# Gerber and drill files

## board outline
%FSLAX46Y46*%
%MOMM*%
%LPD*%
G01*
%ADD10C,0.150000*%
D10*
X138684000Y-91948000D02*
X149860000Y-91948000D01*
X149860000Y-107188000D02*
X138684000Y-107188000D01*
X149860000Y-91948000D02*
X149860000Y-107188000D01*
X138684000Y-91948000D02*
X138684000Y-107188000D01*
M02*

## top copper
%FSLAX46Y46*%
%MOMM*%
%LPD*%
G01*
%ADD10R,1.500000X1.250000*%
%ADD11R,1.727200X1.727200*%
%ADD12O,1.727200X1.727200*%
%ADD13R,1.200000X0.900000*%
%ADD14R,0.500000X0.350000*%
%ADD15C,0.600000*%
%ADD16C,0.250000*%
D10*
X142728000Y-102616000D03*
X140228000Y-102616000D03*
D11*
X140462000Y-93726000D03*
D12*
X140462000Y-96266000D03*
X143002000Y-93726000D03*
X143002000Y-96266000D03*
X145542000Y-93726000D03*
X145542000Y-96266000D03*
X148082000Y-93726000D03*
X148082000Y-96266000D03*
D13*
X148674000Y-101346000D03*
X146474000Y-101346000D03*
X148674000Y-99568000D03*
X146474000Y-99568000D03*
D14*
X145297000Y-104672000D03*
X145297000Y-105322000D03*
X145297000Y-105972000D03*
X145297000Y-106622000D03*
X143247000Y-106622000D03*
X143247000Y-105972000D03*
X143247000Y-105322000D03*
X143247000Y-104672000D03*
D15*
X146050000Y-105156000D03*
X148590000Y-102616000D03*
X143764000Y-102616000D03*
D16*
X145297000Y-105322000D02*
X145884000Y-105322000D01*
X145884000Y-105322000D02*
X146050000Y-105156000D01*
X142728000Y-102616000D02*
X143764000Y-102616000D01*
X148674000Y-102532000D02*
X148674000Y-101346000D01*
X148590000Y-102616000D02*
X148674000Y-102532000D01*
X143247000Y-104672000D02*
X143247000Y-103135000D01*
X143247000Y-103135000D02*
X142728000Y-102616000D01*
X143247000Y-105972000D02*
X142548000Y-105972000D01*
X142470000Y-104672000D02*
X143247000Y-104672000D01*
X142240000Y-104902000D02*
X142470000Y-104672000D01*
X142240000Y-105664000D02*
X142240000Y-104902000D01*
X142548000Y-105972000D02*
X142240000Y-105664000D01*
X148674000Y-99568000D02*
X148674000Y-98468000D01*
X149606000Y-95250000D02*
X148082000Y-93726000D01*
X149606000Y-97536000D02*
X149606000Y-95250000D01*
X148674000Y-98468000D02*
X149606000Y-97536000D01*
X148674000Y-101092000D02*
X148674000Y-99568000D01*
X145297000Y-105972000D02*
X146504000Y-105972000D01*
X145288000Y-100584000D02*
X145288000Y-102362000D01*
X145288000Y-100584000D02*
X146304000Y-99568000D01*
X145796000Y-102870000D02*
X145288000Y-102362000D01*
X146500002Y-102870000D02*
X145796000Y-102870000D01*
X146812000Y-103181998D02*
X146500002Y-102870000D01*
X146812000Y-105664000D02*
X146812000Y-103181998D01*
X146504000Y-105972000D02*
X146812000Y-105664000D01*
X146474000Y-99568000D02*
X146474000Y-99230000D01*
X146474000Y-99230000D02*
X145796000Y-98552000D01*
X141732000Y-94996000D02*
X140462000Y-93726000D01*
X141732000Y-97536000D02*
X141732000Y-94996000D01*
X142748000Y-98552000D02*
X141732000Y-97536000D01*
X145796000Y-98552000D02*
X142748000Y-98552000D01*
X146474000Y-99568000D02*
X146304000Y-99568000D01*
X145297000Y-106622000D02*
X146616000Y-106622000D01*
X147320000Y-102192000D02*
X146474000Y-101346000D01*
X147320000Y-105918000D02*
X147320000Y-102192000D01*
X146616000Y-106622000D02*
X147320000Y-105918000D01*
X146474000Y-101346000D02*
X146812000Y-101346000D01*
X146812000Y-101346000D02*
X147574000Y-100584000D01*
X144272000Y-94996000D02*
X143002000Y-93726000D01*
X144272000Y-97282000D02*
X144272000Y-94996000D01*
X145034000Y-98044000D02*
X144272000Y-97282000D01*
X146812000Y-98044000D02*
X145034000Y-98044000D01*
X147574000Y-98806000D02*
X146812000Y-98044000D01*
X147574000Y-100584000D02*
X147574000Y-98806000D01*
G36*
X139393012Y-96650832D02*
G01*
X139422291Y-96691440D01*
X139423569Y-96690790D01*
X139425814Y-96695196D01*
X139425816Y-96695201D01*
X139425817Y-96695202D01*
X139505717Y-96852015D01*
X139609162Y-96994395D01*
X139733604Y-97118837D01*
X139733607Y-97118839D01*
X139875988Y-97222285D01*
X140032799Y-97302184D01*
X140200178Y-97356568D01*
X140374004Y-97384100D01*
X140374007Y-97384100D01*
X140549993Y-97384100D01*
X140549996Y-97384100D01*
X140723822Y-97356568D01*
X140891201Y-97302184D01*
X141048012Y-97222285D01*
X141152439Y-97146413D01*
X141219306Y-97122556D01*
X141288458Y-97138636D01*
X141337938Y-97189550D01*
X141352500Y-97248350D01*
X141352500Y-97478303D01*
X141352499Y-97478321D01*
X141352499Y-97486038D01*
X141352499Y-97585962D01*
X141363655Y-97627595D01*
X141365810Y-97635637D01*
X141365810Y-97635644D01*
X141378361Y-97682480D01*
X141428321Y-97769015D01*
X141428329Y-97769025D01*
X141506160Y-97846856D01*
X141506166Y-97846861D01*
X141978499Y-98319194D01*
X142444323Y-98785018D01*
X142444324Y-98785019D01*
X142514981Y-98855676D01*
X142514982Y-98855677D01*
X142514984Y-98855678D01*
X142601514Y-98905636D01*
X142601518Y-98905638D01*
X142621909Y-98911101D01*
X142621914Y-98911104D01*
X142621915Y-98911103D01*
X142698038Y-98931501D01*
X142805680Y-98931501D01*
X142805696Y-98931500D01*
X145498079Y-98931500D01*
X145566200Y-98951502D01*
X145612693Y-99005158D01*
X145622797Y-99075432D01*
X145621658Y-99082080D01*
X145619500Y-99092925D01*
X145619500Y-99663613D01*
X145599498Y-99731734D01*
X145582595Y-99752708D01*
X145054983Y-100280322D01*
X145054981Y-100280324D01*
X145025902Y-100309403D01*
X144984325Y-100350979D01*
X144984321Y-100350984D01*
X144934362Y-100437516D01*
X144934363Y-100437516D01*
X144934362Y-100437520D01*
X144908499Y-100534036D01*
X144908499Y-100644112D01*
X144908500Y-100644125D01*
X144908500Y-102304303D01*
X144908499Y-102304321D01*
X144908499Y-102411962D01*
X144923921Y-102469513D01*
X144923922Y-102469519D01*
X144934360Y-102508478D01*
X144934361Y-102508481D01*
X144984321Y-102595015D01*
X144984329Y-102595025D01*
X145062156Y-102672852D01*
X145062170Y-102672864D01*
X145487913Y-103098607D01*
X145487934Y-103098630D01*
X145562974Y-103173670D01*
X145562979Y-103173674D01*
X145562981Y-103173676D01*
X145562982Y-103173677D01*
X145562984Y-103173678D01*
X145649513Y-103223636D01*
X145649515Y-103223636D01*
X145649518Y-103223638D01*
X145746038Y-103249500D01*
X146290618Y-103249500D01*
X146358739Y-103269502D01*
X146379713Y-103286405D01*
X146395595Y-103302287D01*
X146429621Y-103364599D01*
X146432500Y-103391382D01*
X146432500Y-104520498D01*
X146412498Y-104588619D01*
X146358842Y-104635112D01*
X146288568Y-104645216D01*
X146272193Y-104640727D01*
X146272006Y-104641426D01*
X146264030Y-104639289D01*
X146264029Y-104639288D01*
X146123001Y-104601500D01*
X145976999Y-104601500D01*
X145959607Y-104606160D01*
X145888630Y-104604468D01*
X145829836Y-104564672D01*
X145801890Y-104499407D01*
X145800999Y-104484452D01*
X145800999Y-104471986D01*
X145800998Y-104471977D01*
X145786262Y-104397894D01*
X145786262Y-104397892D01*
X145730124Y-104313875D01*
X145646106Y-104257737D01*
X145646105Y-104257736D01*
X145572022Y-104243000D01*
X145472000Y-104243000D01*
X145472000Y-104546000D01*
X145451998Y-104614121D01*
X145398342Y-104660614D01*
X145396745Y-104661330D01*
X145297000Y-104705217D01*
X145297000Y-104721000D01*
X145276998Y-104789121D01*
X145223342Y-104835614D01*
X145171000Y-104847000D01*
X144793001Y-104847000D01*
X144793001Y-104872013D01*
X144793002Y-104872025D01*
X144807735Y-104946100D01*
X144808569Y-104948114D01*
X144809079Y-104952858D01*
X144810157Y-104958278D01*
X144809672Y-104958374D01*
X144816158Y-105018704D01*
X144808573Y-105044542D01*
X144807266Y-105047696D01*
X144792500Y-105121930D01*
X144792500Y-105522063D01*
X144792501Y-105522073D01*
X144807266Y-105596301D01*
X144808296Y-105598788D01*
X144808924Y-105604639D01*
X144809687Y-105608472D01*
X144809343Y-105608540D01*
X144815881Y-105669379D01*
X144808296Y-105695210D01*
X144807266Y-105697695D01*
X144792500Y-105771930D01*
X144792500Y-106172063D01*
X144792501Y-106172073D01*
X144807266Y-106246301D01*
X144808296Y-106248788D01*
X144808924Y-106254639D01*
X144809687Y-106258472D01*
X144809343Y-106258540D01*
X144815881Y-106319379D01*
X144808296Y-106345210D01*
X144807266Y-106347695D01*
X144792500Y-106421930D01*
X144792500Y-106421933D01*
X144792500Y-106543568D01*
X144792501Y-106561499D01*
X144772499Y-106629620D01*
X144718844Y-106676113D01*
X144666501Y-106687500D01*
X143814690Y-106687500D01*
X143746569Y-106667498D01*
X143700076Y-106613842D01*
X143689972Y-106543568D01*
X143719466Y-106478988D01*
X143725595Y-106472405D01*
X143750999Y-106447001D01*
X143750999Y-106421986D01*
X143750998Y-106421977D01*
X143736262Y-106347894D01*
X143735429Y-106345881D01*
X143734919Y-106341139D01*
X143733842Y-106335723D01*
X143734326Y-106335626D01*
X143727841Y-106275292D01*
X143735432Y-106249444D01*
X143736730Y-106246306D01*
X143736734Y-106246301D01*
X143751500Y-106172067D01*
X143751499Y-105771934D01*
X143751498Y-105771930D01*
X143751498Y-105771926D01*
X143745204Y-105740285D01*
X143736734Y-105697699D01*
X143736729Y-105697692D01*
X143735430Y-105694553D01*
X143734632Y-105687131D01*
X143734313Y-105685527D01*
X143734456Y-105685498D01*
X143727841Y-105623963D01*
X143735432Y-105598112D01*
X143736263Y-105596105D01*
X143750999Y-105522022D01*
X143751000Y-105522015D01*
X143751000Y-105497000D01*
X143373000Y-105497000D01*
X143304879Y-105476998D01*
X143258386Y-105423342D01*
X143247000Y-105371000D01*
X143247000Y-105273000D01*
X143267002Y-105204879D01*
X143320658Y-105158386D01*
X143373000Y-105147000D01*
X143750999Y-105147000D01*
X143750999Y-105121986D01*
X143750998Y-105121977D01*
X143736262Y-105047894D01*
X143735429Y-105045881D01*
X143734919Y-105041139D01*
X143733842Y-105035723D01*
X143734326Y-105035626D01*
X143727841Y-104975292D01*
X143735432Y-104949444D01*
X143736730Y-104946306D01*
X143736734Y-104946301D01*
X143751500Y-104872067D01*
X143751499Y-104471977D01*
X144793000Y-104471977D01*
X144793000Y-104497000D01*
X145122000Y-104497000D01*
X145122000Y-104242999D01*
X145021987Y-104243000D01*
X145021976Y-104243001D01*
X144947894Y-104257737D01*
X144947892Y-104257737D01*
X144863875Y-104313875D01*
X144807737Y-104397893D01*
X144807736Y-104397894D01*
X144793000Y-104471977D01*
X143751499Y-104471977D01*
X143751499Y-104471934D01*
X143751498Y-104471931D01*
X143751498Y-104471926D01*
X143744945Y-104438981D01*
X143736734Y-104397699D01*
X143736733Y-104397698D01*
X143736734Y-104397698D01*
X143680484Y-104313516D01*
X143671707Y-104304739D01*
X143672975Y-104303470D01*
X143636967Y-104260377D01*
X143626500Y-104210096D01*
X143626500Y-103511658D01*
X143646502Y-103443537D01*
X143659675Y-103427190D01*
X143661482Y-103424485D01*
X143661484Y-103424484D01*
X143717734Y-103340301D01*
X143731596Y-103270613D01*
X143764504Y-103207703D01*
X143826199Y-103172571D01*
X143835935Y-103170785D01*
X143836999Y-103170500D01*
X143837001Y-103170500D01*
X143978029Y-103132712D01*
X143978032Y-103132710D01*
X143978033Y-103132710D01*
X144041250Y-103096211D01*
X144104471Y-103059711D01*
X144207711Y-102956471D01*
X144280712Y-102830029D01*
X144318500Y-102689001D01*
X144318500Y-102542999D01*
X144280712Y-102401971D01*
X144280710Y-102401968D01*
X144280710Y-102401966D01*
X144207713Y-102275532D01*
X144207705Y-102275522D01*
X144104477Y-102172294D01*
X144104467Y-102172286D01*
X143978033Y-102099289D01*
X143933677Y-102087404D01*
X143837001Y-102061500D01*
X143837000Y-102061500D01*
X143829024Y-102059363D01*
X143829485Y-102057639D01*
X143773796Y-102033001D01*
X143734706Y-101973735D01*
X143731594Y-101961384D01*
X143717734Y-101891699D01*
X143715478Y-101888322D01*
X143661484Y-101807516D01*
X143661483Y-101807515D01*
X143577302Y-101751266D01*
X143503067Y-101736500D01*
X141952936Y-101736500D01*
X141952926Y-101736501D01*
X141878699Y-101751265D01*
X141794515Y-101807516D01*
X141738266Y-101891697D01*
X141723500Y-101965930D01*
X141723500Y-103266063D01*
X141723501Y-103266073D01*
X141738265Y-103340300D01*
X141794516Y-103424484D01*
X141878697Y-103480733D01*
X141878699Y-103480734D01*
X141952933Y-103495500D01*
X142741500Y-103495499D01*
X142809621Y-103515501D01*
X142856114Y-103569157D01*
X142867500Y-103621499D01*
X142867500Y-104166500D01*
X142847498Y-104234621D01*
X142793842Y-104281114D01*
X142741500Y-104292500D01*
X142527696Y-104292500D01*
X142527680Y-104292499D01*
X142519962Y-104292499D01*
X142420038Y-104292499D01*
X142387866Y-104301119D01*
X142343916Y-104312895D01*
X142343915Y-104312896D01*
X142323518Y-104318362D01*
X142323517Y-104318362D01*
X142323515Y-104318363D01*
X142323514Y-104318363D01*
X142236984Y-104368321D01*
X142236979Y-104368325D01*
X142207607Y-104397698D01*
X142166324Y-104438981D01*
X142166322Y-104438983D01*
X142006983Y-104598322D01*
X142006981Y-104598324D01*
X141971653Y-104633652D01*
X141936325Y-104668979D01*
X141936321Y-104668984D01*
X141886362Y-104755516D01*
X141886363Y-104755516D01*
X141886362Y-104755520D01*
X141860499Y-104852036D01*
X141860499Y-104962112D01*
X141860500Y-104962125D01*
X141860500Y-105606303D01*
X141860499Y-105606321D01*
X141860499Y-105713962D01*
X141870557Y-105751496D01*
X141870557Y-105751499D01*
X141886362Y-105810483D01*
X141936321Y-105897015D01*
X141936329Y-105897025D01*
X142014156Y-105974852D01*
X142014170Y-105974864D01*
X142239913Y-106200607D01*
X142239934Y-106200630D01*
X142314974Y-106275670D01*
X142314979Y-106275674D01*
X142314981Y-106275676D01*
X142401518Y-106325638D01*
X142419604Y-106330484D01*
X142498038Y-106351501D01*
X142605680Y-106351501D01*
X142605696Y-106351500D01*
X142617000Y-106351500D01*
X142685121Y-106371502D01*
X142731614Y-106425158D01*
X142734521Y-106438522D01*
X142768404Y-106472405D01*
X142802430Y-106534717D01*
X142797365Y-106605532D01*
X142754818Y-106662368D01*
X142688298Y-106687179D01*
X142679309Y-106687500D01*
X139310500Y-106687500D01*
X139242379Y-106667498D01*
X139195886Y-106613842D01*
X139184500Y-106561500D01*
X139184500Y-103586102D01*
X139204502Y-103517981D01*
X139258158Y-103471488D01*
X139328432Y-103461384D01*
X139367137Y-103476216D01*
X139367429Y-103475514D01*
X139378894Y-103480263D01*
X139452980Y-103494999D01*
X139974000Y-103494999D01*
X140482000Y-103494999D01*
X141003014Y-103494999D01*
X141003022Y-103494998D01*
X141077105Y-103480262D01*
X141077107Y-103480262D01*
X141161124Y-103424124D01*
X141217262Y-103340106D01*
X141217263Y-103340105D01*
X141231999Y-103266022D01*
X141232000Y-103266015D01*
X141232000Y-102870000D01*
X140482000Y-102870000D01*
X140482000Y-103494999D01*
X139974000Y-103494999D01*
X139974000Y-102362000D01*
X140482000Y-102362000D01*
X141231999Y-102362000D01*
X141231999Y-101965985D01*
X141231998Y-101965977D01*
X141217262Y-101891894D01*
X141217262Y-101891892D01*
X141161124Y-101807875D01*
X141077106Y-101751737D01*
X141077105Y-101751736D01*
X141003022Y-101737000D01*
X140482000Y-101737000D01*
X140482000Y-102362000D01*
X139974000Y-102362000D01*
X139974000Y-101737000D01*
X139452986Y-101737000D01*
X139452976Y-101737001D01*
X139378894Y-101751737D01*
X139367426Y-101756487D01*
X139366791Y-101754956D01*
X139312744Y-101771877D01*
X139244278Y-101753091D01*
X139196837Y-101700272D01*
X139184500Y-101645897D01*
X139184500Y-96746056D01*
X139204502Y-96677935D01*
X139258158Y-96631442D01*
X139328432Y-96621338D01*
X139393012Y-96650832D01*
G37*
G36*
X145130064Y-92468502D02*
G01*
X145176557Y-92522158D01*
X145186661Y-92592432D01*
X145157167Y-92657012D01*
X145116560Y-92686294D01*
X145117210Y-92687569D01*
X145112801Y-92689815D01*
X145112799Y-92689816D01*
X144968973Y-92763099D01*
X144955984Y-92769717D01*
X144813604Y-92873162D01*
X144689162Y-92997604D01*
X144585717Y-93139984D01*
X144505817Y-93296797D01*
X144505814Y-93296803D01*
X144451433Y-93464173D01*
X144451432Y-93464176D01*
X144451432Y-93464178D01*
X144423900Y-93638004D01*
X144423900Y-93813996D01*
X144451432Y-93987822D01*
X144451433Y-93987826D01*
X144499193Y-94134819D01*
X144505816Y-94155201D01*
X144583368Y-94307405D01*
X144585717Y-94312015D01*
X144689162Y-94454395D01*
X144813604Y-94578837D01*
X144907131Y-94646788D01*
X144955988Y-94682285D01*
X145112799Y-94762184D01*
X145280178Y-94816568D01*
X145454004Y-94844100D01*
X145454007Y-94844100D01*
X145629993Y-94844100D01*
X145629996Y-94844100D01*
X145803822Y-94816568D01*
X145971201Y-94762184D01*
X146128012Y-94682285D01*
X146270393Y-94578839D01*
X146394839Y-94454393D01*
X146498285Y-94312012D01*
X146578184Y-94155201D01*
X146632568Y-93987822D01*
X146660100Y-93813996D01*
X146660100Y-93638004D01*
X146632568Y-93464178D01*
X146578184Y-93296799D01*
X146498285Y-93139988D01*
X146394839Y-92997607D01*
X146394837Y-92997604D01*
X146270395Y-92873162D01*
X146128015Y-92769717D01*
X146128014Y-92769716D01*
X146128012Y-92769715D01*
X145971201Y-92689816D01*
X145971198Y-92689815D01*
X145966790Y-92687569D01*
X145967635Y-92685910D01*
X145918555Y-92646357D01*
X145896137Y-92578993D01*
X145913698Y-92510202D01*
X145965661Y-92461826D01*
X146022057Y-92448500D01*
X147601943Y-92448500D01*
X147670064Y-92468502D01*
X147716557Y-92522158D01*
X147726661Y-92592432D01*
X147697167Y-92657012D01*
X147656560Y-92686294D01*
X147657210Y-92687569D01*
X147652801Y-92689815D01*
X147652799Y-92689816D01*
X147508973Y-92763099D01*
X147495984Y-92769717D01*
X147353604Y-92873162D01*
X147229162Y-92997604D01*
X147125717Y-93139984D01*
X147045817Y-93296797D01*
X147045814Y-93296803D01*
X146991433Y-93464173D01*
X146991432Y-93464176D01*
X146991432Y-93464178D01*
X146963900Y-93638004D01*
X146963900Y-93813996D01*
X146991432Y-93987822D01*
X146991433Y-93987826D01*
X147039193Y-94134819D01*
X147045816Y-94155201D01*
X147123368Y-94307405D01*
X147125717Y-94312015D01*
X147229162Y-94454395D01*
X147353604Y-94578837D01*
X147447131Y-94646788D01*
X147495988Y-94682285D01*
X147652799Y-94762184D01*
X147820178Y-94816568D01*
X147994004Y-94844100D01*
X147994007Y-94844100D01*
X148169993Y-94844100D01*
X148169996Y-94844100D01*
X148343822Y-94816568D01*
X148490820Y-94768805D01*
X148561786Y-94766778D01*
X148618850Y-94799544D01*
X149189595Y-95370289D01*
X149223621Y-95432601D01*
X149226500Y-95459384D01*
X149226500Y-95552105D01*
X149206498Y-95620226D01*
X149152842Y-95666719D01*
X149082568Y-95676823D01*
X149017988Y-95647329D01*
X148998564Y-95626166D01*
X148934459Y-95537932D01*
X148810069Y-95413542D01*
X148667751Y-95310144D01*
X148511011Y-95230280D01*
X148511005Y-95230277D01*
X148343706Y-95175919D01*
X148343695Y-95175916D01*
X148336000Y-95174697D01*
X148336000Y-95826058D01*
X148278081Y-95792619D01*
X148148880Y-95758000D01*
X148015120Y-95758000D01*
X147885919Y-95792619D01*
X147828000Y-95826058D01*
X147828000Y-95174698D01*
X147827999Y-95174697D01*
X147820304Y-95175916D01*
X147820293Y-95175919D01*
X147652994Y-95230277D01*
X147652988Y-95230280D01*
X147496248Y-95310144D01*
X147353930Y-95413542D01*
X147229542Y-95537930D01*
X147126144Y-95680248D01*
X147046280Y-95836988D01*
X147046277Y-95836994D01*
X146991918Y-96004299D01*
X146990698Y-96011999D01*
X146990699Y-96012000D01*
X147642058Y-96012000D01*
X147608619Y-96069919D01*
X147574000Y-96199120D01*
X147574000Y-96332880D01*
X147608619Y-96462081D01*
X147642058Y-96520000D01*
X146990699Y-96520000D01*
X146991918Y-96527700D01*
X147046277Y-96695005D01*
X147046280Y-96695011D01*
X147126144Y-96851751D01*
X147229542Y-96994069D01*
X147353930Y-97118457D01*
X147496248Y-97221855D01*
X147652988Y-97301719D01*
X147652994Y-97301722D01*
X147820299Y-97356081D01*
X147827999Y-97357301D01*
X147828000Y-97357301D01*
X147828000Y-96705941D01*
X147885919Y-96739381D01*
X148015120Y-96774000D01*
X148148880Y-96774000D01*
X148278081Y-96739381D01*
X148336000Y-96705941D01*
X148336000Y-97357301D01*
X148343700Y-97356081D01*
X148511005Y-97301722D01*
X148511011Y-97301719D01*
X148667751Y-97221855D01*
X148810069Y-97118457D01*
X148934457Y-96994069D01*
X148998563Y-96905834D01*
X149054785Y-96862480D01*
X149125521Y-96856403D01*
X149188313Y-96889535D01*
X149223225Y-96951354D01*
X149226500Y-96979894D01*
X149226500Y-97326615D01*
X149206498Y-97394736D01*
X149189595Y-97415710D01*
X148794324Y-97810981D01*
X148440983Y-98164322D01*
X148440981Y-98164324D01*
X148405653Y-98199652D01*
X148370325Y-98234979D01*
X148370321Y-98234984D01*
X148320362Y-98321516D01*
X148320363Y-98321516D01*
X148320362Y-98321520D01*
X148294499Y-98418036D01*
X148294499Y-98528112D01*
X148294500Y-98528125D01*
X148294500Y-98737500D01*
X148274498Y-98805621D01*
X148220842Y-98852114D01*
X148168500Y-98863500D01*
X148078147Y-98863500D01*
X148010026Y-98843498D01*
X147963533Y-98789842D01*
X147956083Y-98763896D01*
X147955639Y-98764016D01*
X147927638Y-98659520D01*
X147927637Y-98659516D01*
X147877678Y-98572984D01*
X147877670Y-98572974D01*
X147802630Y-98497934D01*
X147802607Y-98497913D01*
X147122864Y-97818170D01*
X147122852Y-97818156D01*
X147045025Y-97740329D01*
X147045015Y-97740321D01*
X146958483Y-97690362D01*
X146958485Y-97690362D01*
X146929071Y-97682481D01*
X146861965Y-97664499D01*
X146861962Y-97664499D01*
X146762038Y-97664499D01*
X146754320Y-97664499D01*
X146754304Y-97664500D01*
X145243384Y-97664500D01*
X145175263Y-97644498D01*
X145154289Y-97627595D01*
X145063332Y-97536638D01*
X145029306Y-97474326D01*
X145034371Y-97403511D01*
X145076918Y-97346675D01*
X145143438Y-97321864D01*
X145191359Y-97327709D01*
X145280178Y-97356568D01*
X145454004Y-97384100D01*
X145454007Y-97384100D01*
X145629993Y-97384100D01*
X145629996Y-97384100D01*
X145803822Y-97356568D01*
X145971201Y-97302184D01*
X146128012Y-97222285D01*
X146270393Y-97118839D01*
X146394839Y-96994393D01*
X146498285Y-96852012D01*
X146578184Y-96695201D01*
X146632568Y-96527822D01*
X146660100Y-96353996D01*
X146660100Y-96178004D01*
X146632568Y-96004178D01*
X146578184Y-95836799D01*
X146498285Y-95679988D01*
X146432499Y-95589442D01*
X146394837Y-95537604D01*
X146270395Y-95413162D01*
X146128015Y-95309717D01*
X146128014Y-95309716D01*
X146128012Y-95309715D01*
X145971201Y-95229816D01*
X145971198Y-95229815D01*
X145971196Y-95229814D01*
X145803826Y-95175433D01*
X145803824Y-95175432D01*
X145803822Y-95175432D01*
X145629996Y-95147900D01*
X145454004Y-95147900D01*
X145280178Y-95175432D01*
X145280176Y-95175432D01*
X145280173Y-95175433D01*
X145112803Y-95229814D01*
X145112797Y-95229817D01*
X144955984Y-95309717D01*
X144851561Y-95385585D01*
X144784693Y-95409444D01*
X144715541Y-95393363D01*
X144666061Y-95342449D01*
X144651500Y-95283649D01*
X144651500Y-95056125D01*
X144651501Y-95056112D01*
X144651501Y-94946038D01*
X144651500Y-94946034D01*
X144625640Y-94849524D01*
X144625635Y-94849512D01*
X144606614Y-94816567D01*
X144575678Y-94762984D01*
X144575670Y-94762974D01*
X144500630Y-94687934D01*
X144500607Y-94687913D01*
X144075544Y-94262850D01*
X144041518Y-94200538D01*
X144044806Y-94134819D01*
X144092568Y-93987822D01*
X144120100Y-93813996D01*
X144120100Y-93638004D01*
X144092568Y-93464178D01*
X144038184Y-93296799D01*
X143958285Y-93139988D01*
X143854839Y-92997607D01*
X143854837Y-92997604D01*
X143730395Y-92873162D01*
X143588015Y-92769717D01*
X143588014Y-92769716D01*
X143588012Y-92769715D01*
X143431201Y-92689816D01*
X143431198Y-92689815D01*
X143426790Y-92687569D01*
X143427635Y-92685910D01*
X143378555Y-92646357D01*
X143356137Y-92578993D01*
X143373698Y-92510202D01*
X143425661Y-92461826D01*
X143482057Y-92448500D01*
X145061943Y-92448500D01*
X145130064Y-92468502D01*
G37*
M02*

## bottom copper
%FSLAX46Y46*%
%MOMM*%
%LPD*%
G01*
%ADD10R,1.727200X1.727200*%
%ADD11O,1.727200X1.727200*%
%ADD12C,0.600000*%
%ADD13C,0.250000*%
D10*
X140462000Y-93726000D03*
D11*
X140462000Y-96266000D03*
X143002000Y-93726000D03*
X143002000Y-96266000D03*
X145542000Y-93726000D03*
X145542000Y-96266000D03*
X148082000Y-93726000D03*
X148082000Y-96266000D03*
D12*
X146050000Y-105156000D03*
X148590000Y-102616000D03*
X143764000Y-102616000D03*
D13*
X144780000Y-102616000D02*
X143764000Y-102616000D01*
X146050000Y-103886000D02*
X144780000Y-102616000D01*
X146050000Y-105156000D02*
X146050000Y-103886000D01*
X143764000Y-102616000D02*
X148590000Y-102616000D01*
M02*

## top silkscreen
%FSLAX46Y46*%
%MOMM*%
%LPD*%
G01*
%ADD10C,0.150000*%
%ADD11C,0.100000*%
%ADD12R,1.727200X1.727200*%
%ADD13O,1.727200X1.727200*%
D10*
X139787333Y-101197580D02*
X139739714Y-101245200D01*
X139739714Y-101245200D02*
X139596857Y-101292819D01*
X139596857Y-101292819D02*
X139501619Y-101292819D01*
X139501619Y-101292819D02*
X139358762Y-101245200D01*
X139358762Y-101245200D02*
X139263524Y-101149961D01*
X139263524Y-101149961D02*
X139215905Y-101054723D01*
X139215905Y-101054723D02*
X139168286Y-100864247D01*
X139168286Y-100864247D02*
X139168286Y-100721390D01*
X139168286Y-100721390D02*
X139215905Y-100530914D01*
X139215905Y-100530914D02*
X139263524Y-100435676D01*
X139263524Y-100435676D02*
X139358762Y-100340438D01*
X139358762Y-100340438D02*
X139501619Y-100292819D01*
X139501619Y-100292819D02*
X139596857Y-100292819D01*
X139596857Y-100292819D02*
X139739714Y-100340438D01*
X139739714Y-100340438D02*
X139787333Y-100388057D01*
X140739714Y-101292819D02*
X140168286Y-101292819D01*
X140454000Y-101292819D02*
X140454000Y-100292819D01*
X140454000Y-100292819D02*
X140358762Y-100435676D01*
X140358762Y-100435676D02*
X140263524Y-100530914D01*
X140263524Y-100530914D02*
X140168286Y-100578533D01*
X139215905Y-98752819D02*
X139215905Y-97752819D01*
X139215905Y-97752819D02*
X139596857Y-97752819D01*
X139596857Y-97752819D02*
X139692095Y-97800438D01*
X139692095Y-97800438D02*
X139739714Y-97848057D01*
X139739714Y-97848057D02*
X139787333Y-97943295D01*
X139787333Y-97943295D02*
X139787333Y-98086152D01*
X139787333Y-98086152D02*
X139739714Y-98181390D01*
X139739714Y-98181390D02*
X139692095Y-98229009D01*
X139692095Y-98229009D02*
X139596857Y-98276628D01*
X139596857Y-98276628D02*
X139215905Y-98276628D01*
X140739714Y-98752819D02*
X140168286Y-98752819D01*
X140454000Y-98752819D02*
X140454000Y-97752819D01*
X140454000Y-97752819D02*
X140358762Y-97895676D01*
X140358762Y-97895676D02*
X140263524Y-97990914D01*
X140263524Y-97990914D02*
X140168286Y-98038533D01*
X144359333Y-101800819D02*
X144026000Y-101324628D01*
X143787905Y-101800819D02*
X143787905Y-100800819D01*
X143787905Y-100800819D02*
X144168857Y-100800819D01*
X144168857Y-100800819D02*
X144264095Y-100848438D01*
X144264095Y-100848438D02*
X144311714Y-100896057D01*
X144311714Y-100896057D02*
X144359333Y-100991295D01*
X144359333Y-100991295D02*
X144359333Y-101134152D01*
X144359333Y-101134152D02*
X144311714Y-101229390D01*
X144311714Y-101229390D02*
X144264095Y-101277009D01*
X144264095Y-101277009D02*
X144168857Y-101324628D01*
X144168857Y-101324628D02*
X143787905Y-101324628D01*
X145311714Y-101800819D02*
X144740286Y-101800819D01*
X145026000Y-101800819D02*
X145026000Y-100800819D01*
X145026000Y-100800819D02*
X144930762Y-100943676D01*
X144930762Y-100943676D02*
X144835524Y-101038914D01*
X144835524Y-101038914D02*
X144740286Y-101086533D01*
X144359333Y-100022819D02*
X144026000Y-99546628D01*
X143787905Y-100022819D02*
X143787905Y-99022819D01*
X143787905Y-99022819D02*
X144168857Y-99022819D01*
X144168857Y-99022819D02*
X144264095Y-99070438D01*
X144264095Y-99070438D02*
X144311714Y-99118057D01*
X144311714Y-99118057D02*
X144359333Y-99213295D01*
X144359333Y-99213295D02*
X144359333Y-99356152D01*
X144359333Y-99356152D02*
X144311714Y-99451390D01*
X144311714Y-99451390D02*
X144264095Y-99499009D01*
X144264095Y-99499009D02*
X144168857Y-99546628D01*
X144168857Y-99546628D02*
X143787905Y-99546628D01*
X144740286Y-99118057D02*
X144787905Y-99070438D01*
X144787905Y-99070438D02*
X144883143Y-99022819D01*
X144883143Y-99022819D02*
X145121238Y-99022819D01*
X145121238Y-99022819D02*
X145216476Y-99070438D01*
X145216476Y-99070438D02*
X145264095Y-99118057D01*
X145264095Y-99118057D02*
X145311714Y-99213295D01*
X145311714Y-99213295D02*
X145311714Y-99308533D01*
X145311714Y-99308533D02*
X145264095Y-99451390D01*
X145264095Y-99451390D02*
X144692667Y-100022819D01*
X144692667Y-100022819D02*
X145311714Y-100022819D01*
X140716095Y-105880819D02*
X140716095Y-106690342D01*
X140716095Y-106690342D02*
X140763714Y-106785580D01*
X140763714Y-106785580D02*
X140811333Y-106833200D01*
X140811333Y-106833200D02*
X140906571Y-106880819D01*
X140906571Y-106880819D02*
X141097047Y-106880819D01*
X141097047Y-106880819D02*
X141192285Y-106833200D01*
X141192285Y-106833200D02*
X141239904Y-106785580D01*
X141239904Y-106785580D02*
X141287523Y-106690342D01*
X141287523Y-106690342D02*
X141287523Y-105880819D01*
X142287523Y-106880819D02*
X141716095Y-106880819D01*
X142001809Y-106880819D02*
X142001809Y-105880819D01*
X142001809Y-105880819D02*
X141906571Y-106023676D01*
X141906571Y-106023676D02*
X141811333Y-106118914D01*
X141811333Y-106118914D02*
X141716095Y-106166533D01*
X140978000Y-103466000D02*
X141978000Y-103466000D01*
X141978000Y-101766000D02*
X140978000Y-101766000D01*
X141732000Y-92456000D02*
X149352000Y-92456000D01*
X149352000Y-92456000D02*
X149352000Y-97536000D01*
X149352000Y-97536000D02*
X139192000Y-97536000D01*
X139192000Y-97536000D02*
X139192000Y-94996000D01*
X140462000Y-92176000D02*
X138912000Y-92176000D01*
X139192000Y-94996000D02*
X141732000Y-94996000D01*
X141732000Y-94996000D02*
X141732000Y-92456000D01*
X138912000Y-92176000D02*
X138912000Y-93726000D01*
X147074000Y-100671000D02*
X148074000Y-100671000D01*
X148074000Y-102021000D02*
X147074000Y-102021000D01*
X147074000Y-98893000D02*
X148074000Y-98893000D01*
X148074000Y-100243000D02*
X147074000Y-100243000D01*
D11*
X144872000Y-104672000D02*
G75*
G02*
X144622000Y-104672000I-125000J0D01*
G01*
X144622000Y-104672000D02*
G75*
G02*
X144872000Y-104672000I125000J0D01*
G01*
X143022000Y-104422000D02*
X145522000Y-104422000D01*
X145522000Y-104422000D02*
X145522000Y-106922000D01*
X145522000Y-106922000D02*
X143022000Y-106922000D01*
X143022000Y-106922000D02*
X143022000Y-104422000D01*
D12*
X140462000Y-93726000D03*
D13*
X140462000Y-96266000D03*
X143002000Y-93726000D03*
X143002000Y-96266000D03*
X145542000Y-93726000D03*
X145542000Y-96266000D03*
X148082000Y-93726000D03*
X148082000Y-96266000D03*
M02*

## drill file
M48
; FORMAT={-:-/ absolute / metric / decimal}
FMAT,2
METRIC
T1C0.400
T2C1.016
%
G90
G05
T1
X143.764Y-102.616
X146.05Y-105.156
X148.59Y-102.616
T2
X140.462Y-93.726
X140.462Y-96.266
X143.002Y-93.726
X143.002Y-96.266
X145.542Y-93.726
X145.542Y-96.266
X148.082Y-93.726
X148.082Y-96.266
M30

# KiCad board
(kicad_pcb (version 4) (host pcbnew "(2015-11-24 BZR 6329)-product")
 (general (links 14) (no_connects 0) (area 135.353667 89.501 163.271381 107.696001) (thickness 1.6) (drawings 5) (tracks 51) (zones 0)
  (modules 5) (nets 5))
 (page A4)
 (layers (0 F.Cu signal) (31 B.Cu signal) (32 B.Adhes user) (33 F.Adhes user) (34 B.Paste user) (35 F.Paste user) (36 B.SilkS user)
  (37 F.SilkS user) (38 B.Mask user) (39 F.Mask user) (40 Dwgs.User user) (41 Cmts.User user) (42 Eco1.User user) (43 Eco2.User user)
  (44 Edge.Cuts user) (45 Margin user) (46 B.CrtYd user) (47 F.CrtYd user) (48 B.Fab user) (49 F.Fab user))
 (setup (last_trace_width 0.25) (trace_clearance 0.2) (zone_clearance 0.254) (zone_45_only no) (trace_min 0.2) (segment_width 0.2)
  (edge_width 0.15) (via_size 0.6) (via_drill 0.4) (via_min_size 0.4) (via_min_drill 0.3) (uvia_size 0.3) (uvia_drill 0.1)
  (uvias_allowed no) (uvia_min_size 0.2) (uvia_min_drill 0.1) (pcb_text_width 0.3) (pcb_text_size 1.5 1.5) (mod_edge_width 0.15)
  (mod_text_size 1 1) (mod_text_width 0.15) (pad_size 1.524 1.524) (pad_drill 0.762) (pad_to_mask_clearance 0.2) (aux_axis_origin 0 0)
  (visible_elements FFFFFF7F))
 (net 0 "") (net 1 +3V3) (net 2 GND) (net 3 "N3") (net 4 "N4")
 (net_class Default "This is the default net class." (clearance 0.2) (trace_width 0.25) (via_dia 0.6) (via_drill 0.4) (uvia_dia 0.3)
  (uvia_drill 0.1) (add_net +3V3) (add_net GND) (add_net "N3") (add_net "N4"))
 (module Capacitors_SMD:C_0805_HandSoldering (layer F.Cu) (at 141.478 102.616 180)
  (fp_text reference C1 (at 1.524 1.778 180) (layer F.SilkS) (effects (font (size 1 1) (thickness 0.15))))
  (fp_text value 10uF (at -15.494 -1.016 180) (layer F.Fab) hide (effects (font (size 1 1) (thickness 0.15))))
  (fp_line (start 0.5 -0.85) (end -0.5 -0.85) (layer F.SilkS) (width 0.15))
  (fp_line (start -0.5 0.85) (end 0.5 0.85) (layer F.SilkS) (width 0.15))
  (pad 1 smd rect (at -1.25 0 180) (size 1.5 1.25) (layers F.Cu F.Paste F.Mask) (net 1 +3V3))
  (pad 2 smd rect (at 1.25 0 180) (size 1.5 1.25) (layers F.Cu F.Paste F.Mask) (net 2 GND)))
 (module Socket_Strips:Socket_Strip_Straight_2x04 (layer F.Cu) (at 140.462 93.726)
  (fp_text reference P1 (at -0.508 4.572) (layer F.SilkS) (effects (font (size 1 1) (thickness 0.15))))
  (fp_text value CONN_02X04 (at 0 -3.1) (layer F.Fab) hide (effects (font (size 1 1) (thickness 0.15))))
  (fp_line (start 1.27 -1.27) (end 8.89 -1.27) (layer F.SilkS) (width 0.15))
  (fp_line (start 8.89 -1.27) (end 8.89 3.81) (layer F.SilkS) (width 0.15))
  (fp_line (start 8.89 3.81) (end -1.27 3.81) (layer F.SilkS) (width 0.15))
  (fp_line (start -1.27 3.81) (end -1.27 1.27) (layer F.SilkS) (width 0.15))
  (fp_line (start 0 -1.55) (end -1.55 -1.55) (layer F.SilkS) (width 0.15))
  (fp_line (start -1.27 1.27) (end 1.27 1.27) (layer F.SilkS) (width 0.15))
  (fp_line (start 1.27 1.27) (end 1.27 -1.27) (layer F.SilkS) (width 0.15))
  (fp_line (start -1.55 -1.55) (end -1.55 0) (layer F.SilkS) (width 0.15))
  (pad 1 thru_hole rect (at 0 0) (size 1.7272 1.7272) (drill 1.016) (layers *.Cu *.Mask F.SilkS) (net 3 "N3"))
  (pad 2 thru_hole oval (at 0 2.54) (size 1.7272 1.7272) (drill 1.016) (layers *.Cu *.Mask F.SilkS))
  (pad 3 thru_hole oval (at 2.54 0) (size 1.7272 1.7272) (drill 1.016) (layers *.Cu *.Mask F.SilkS) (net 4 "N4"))
  (pad 4 thru_hole oval (at 2.54 2.54) (size 1.7272 1.7272) (drill 1.016) (layers *.Cu *.Mask F.SilkS))
  (pad 5 thru_hole oval (at 5.08 0) (size 1.7272 1.7272) (drill 1.016) (layers *.Cu *.Mask F.SilkS))
  (pad 6 thru_hole oval (at 5.08 2.54) (size 1.7272 1.7272) (drill 1.016) (layers *.Cu *.Mask F.SilkS))
  (pad 7 thru_hole oval (at 7.62 0) (size 1.7272 1.7272) (drill 1.016) (layers *.Cu *.Mask F.SilkS) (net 1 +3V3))
  (pad 8 thru_hole oval (at 7.62 2.54) (size 1.7272 1.7272) (drill 1.016) (layers *.Cu *.Mask F.SilkS) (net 2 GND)))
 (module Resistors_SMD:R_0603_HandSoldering (layer F.Cu) (at 147.574 101.346 180)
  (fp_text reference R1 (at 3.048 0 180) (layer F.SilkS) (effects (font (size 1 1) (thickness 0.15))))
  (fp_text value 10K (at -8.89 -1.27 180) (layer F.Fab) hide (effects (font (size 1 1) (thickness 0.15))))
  (fp_line (start 0.5 0.675) (end -0.5 0.675) (layer F.SilkS) (width 0.15))
  (fp_line (start -0.5 -0.675) (end 0.5 -0.675) (layer F.SilkS) (width 0.15))
  (pad 1 smd rect (at -1.1 0 180) (size 1.2 0.9) (layers F.Cu F.Paste F.Mask) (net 1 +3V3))
  (pad 2 smd rect (at 1.1 0 180) (size 1.2 0.9) (layers F.Cu F.Paste F.Mask) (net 4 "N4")))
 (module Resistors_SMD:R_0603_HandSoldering (layer F.Cu) (at 147.574 99.568 180)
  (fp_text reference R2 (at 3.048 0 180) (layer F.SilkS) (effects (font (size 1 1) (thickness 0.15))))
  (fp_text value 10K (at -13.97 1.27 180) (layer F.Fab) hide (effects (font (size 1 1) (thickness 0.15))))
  (fp_line (start 0.5 0.675) (end -0.5 0.675) (layer F.SilkS) (width 0.15))
  (fp_line (start -0.5 -0.675) (end 0.5 -0.675) (layer F.SilkS) (width 0.15))
  (pad 1 smd rect (at -1.1 0 180) (size 1.2 0.9) (layers F.Cu F.Paste F.Mask) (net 1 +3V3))
  (pad 2 smd rect (at 1.1 0 180) (size 1.2 0.9) (layers F.Cu F.Paste F.Mask) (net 3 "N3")))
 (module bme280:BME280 (layer F.Cu) (at 144.272 106.172)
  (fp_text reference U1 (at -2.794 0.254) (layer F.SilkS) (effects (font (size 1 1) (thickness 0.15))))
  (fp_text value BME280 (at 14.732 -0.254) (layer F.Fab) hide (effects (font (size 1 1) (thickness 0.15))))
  (fp_circle (center 0.475 -1.5) (end 0.55 -1.4) (layer F.SilkS) (width 0.1))
  (fp_line (start -1.25 -1.75) (end 1.25 -1.75) (layer F.SilkS) (width 0.1))
  (fp_line (start 1.25 -1.75) (end 1.25 0.75) (layer F.SilkS) (width 0.1))
  (fp_line (start 1.25 0.75) (end -1.25 0.75) (layer F.SilkS) (width 0.1))
  (fp_line (start -1.25 0.75) (end -1.25 -1.75) (layer F.SilkS) (width 0.1))
  (pad 1 smd rect (at 1.025 -1.5) (size 0.5 0.35) (layers F.Cu F.Paste F.Mask) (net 2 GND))
  (pad 2 smd rect (at 1.025 -0.85) (size 0.5 0.35) (layers F.Cu F.Paste F.Mask) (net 1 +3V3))
  (pad 3 smd rect (at 1.025 -0.2) (size 0.5 0.35) (layers F.Cu F.Paste F.Mask) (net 3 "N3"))
  (pad 4 smd rect (at 1.025 0.45) (size 0.5 0.35) (layers F.Cu F.Paste F.Mask) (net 4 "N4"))
  (pad 5 smd rect (at -1.025 0.45) (size 0.5 0.35) (layers F.Cu F.Paste F.Mask) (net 2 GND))
  (pad 6 smd rect (at -1.025 -0.2) (size 0.5 0.35) (layers F.Cu F.Paste F.Mask) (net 1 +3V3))
  (pad 7 smd rect (at -1.025 -0.85) (size 0.5 0.35) (layers F.Cu F.Paste F.Mask) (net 2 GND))
  (pad 8 smd rect (at -1.025 -1.5) (size 0.5 0.35) (layers F.Cu F.Paste F.Mask) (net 1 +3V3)))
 (gr_line (start 138.684 91.948) (end 149.86 91.948) (angle 90) (layer Edge.Cuts) (width 0.15))
 (gr_line (start 149.86 107.188) (end 138.684 107.188) (angle 90) (layer Edge.Cuts) (width 0.15))
 (gr_line (start 149.86 91.948) (end 149.86 107.188) (angle 90) (layer Edge.Cuts) (width 0.15))
 (gr_line (start 138.684 91.948) (end 138.684 107.188) (angle 90) (layer Edge.Cuts) (width 0.15))
 (segment (start 145.297 105.322) (end 145.884 105.322) (width 0.25) (layer F.Cu) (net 1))
 (segment (start 144.78 102.616) (end 143.764 102.616) (width 0.25) (layer B.Cu) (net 1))
 (segment (start 146.05 103.886) (end 144.78 102.616) (width 0.25) (layer B.Cu) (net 1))
 (segment (start 146.05 105.156) (end 146.05 103.886) (width 0.25) (layer B.Cu) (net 1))
 (via (at 146.05 105.156) (size 0.6) (drill 0.4) (layers F.Cu B.Cu) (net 1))
 (segment (start 145.884 105.322) (end 146.05 105.156) (width 0.25) (layer F.Cu) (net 1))
 (segment (start 142.728 102.616) (end 143.764 102.616) (width 0.25) (layer F.Cu) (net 1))
 (segment (start 148.674 102.532) (end 148.674 101.346) (width 0.25) (layer F.Cu) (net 1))
 (segment (start 148.59 102.616) (end 148.674 102.532) (width 0.25) (layer F.Cu) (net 1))
 (via (at 148.59 102.616) (size 0.6) (drill 0.4) (layers F.Cu B.Cu) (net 1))
 (segment (start 143.764 102.616) (end 148.59 102.616) (width 0.25) (layer B.Cu) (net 1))
 (via (at 143.764 102.616) (size 0.6) (drill 0.4) (layers F.Cu B.Cu) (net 1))
 (segment (start 143.247 104.672) (end 143.247 103.135) (width 0.25) (layer F.Cu) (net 1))
 (segment (start 143.247 103.135) (end 142.728 102.616) (width 0.25) (layer F.Cu) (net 1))
 (segment (start 143.247 105.972) (end 142.548 105.972) (width 0.25) (layer F.Cu) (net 1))
 (segment (start 142.47 104.672) (end 143.247 104.672) (width 0.25) (layer F.Cu) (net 1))
 (segment (start 142.24 104.902) (end 142.47 104.672) (width 0.25) (layer F.Cu) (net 1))
 (segment (start 142.24 105.664) (end 142.24 104.902) (width 0.25) (layer F.Cu) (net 1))
 (segment (start 142.548 105.972) (end 142.24 105.664) (width 0.25) (layer F.Cu) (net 1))
 (segment (start 148.674 99.568) (end 148.674 98.468) (width 0.25) (layer F.Cu) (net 1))
 (segment (start 149.606 95.25) (end 148.082 93.726) (width 0.25) (layer F.Cu) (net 1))
 (segment (start 149.606 97.536) (end 149.606 95.25) (width 0.25) (layer F.Cu) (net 1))
 (segment (start 148.674 98.468) (end 149.606 97.536) (width 0.25) (layer F.Cu) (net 1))
 (segment (start 148.674 101.092) (end 148.674 99.568) (width 0.25) (layer F.Cu) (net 1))
 (segment (start 145.297 105.972) (end 146.504 105.972) (width 0.25) (layer F.Cu) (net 3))
 (segment (start 145.288 100.584) (end 145.288 102.362) (width 0.25) (layer F.Cu) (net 3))
 (segment (start 145.288 100.584) (end 146.304 99.568) (width 0.25) (layer F.Cu) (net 3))
 (segment (start 145.796 102.87) (end 145.288 102.362) (width 0.25) (layer F.Cu) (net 3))
 (segment (start 146.500002 102.87) (end 145.796 102.87) (width 0.25) (layer F.Cu) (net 3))
 (segment (start 146.812 103.181998) (end 146.500002 102.87) (width 0.25) (layer F.Cu) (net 3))
 (segment (start 146.812 105.664) (end 146.812 103.181998) (width 0.25) (layer F.Cu) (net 3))
 (segment (start 146.504 105.972) (end 146.812 105.664) (width 0.25) (layer F.Cu) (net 3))
 (segment (start 146.474 99.568) (end 146.474 99.23) (width 0.25) (layer F.Cu) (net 3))
 (segment (start 146.474 99.23) (end 145.796 98.552) (width 0.25) (layer F.Cu) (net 3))
 (segment (start 141.732 94.996) (end 140.462 93.726) (width 0.25) (layer F.Cu) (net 3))
 (segment (start 141.732 97.536) (end 141.732 94.996) (width 0.25) (layer F.Cu) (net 3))
 (segment (start 142.748 98.552) (end 141.732 97.536) (width 0.25) (layer F.Cu) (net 3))
 (segment (start 145.796 98.552) (end 142.748 98.552) (width 0.25) (layer F.Cu) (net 3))
 (segment (start 146.474 99.568) (end 146.304 99.568) (width 0.25) (layer F.Cu) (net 3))
 (segment (start 145.297 106.622) (end 146.616 106.622) (width 0.25) (layer F.Cu) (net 4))
 (segment (start 147.32 102.192) (end 146.474 101.346) (width 0.25) (layer F.Cu) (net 4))
 (segment (start 147.32 105.918) (end 147.32 102.192) (width 0.25) (layer F.Cu) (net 4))
 (segment (start 146.616 106.622) (end 147.32 105.918) (width 0.25) (layer F.Cu) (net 4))
 (segment (start 146.474 101.346) (end 146.812 101.346) (width 0.25) (layer F.Cu) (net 4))
 (segment (start 146.812 101.346) (end 147.574 100.584) (width 0.25) (layer F.Cu) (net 4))
 (segment (start 144.272 94.996) (end 143.002 93.726) (width 0.25) (layer F.Cu) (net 4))
 (segment (start 144.272 97.282) (end 144.272 94.996) (width 0.25) (layer F.Cu) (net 4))
 (segment (start 145.034 98.044) (end 144.272 97.282) (width 0.25) (layer F.Cu) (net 4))
 (segment (start 146.812 98.044) (end 145.034 98.044) (width 0.25) (layer F.Cu) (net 4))
 (segment (start 147.574 98.806) (end 146.812 98.044) (width 0.25) (layer F.Cu) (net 4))
 (segment (start 147.574 100.584) (end 147.574 98.806) (width 0.25) (layer F.Cu) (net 4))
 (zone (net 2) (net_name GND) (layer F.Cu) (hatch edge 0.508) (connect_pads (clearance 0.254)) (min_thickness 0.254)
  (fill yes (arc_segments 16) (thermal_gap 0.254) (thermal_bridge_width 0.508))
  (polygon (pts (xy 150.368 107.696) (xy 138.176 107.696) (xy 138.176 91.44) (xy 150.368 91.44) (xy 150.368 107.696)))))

